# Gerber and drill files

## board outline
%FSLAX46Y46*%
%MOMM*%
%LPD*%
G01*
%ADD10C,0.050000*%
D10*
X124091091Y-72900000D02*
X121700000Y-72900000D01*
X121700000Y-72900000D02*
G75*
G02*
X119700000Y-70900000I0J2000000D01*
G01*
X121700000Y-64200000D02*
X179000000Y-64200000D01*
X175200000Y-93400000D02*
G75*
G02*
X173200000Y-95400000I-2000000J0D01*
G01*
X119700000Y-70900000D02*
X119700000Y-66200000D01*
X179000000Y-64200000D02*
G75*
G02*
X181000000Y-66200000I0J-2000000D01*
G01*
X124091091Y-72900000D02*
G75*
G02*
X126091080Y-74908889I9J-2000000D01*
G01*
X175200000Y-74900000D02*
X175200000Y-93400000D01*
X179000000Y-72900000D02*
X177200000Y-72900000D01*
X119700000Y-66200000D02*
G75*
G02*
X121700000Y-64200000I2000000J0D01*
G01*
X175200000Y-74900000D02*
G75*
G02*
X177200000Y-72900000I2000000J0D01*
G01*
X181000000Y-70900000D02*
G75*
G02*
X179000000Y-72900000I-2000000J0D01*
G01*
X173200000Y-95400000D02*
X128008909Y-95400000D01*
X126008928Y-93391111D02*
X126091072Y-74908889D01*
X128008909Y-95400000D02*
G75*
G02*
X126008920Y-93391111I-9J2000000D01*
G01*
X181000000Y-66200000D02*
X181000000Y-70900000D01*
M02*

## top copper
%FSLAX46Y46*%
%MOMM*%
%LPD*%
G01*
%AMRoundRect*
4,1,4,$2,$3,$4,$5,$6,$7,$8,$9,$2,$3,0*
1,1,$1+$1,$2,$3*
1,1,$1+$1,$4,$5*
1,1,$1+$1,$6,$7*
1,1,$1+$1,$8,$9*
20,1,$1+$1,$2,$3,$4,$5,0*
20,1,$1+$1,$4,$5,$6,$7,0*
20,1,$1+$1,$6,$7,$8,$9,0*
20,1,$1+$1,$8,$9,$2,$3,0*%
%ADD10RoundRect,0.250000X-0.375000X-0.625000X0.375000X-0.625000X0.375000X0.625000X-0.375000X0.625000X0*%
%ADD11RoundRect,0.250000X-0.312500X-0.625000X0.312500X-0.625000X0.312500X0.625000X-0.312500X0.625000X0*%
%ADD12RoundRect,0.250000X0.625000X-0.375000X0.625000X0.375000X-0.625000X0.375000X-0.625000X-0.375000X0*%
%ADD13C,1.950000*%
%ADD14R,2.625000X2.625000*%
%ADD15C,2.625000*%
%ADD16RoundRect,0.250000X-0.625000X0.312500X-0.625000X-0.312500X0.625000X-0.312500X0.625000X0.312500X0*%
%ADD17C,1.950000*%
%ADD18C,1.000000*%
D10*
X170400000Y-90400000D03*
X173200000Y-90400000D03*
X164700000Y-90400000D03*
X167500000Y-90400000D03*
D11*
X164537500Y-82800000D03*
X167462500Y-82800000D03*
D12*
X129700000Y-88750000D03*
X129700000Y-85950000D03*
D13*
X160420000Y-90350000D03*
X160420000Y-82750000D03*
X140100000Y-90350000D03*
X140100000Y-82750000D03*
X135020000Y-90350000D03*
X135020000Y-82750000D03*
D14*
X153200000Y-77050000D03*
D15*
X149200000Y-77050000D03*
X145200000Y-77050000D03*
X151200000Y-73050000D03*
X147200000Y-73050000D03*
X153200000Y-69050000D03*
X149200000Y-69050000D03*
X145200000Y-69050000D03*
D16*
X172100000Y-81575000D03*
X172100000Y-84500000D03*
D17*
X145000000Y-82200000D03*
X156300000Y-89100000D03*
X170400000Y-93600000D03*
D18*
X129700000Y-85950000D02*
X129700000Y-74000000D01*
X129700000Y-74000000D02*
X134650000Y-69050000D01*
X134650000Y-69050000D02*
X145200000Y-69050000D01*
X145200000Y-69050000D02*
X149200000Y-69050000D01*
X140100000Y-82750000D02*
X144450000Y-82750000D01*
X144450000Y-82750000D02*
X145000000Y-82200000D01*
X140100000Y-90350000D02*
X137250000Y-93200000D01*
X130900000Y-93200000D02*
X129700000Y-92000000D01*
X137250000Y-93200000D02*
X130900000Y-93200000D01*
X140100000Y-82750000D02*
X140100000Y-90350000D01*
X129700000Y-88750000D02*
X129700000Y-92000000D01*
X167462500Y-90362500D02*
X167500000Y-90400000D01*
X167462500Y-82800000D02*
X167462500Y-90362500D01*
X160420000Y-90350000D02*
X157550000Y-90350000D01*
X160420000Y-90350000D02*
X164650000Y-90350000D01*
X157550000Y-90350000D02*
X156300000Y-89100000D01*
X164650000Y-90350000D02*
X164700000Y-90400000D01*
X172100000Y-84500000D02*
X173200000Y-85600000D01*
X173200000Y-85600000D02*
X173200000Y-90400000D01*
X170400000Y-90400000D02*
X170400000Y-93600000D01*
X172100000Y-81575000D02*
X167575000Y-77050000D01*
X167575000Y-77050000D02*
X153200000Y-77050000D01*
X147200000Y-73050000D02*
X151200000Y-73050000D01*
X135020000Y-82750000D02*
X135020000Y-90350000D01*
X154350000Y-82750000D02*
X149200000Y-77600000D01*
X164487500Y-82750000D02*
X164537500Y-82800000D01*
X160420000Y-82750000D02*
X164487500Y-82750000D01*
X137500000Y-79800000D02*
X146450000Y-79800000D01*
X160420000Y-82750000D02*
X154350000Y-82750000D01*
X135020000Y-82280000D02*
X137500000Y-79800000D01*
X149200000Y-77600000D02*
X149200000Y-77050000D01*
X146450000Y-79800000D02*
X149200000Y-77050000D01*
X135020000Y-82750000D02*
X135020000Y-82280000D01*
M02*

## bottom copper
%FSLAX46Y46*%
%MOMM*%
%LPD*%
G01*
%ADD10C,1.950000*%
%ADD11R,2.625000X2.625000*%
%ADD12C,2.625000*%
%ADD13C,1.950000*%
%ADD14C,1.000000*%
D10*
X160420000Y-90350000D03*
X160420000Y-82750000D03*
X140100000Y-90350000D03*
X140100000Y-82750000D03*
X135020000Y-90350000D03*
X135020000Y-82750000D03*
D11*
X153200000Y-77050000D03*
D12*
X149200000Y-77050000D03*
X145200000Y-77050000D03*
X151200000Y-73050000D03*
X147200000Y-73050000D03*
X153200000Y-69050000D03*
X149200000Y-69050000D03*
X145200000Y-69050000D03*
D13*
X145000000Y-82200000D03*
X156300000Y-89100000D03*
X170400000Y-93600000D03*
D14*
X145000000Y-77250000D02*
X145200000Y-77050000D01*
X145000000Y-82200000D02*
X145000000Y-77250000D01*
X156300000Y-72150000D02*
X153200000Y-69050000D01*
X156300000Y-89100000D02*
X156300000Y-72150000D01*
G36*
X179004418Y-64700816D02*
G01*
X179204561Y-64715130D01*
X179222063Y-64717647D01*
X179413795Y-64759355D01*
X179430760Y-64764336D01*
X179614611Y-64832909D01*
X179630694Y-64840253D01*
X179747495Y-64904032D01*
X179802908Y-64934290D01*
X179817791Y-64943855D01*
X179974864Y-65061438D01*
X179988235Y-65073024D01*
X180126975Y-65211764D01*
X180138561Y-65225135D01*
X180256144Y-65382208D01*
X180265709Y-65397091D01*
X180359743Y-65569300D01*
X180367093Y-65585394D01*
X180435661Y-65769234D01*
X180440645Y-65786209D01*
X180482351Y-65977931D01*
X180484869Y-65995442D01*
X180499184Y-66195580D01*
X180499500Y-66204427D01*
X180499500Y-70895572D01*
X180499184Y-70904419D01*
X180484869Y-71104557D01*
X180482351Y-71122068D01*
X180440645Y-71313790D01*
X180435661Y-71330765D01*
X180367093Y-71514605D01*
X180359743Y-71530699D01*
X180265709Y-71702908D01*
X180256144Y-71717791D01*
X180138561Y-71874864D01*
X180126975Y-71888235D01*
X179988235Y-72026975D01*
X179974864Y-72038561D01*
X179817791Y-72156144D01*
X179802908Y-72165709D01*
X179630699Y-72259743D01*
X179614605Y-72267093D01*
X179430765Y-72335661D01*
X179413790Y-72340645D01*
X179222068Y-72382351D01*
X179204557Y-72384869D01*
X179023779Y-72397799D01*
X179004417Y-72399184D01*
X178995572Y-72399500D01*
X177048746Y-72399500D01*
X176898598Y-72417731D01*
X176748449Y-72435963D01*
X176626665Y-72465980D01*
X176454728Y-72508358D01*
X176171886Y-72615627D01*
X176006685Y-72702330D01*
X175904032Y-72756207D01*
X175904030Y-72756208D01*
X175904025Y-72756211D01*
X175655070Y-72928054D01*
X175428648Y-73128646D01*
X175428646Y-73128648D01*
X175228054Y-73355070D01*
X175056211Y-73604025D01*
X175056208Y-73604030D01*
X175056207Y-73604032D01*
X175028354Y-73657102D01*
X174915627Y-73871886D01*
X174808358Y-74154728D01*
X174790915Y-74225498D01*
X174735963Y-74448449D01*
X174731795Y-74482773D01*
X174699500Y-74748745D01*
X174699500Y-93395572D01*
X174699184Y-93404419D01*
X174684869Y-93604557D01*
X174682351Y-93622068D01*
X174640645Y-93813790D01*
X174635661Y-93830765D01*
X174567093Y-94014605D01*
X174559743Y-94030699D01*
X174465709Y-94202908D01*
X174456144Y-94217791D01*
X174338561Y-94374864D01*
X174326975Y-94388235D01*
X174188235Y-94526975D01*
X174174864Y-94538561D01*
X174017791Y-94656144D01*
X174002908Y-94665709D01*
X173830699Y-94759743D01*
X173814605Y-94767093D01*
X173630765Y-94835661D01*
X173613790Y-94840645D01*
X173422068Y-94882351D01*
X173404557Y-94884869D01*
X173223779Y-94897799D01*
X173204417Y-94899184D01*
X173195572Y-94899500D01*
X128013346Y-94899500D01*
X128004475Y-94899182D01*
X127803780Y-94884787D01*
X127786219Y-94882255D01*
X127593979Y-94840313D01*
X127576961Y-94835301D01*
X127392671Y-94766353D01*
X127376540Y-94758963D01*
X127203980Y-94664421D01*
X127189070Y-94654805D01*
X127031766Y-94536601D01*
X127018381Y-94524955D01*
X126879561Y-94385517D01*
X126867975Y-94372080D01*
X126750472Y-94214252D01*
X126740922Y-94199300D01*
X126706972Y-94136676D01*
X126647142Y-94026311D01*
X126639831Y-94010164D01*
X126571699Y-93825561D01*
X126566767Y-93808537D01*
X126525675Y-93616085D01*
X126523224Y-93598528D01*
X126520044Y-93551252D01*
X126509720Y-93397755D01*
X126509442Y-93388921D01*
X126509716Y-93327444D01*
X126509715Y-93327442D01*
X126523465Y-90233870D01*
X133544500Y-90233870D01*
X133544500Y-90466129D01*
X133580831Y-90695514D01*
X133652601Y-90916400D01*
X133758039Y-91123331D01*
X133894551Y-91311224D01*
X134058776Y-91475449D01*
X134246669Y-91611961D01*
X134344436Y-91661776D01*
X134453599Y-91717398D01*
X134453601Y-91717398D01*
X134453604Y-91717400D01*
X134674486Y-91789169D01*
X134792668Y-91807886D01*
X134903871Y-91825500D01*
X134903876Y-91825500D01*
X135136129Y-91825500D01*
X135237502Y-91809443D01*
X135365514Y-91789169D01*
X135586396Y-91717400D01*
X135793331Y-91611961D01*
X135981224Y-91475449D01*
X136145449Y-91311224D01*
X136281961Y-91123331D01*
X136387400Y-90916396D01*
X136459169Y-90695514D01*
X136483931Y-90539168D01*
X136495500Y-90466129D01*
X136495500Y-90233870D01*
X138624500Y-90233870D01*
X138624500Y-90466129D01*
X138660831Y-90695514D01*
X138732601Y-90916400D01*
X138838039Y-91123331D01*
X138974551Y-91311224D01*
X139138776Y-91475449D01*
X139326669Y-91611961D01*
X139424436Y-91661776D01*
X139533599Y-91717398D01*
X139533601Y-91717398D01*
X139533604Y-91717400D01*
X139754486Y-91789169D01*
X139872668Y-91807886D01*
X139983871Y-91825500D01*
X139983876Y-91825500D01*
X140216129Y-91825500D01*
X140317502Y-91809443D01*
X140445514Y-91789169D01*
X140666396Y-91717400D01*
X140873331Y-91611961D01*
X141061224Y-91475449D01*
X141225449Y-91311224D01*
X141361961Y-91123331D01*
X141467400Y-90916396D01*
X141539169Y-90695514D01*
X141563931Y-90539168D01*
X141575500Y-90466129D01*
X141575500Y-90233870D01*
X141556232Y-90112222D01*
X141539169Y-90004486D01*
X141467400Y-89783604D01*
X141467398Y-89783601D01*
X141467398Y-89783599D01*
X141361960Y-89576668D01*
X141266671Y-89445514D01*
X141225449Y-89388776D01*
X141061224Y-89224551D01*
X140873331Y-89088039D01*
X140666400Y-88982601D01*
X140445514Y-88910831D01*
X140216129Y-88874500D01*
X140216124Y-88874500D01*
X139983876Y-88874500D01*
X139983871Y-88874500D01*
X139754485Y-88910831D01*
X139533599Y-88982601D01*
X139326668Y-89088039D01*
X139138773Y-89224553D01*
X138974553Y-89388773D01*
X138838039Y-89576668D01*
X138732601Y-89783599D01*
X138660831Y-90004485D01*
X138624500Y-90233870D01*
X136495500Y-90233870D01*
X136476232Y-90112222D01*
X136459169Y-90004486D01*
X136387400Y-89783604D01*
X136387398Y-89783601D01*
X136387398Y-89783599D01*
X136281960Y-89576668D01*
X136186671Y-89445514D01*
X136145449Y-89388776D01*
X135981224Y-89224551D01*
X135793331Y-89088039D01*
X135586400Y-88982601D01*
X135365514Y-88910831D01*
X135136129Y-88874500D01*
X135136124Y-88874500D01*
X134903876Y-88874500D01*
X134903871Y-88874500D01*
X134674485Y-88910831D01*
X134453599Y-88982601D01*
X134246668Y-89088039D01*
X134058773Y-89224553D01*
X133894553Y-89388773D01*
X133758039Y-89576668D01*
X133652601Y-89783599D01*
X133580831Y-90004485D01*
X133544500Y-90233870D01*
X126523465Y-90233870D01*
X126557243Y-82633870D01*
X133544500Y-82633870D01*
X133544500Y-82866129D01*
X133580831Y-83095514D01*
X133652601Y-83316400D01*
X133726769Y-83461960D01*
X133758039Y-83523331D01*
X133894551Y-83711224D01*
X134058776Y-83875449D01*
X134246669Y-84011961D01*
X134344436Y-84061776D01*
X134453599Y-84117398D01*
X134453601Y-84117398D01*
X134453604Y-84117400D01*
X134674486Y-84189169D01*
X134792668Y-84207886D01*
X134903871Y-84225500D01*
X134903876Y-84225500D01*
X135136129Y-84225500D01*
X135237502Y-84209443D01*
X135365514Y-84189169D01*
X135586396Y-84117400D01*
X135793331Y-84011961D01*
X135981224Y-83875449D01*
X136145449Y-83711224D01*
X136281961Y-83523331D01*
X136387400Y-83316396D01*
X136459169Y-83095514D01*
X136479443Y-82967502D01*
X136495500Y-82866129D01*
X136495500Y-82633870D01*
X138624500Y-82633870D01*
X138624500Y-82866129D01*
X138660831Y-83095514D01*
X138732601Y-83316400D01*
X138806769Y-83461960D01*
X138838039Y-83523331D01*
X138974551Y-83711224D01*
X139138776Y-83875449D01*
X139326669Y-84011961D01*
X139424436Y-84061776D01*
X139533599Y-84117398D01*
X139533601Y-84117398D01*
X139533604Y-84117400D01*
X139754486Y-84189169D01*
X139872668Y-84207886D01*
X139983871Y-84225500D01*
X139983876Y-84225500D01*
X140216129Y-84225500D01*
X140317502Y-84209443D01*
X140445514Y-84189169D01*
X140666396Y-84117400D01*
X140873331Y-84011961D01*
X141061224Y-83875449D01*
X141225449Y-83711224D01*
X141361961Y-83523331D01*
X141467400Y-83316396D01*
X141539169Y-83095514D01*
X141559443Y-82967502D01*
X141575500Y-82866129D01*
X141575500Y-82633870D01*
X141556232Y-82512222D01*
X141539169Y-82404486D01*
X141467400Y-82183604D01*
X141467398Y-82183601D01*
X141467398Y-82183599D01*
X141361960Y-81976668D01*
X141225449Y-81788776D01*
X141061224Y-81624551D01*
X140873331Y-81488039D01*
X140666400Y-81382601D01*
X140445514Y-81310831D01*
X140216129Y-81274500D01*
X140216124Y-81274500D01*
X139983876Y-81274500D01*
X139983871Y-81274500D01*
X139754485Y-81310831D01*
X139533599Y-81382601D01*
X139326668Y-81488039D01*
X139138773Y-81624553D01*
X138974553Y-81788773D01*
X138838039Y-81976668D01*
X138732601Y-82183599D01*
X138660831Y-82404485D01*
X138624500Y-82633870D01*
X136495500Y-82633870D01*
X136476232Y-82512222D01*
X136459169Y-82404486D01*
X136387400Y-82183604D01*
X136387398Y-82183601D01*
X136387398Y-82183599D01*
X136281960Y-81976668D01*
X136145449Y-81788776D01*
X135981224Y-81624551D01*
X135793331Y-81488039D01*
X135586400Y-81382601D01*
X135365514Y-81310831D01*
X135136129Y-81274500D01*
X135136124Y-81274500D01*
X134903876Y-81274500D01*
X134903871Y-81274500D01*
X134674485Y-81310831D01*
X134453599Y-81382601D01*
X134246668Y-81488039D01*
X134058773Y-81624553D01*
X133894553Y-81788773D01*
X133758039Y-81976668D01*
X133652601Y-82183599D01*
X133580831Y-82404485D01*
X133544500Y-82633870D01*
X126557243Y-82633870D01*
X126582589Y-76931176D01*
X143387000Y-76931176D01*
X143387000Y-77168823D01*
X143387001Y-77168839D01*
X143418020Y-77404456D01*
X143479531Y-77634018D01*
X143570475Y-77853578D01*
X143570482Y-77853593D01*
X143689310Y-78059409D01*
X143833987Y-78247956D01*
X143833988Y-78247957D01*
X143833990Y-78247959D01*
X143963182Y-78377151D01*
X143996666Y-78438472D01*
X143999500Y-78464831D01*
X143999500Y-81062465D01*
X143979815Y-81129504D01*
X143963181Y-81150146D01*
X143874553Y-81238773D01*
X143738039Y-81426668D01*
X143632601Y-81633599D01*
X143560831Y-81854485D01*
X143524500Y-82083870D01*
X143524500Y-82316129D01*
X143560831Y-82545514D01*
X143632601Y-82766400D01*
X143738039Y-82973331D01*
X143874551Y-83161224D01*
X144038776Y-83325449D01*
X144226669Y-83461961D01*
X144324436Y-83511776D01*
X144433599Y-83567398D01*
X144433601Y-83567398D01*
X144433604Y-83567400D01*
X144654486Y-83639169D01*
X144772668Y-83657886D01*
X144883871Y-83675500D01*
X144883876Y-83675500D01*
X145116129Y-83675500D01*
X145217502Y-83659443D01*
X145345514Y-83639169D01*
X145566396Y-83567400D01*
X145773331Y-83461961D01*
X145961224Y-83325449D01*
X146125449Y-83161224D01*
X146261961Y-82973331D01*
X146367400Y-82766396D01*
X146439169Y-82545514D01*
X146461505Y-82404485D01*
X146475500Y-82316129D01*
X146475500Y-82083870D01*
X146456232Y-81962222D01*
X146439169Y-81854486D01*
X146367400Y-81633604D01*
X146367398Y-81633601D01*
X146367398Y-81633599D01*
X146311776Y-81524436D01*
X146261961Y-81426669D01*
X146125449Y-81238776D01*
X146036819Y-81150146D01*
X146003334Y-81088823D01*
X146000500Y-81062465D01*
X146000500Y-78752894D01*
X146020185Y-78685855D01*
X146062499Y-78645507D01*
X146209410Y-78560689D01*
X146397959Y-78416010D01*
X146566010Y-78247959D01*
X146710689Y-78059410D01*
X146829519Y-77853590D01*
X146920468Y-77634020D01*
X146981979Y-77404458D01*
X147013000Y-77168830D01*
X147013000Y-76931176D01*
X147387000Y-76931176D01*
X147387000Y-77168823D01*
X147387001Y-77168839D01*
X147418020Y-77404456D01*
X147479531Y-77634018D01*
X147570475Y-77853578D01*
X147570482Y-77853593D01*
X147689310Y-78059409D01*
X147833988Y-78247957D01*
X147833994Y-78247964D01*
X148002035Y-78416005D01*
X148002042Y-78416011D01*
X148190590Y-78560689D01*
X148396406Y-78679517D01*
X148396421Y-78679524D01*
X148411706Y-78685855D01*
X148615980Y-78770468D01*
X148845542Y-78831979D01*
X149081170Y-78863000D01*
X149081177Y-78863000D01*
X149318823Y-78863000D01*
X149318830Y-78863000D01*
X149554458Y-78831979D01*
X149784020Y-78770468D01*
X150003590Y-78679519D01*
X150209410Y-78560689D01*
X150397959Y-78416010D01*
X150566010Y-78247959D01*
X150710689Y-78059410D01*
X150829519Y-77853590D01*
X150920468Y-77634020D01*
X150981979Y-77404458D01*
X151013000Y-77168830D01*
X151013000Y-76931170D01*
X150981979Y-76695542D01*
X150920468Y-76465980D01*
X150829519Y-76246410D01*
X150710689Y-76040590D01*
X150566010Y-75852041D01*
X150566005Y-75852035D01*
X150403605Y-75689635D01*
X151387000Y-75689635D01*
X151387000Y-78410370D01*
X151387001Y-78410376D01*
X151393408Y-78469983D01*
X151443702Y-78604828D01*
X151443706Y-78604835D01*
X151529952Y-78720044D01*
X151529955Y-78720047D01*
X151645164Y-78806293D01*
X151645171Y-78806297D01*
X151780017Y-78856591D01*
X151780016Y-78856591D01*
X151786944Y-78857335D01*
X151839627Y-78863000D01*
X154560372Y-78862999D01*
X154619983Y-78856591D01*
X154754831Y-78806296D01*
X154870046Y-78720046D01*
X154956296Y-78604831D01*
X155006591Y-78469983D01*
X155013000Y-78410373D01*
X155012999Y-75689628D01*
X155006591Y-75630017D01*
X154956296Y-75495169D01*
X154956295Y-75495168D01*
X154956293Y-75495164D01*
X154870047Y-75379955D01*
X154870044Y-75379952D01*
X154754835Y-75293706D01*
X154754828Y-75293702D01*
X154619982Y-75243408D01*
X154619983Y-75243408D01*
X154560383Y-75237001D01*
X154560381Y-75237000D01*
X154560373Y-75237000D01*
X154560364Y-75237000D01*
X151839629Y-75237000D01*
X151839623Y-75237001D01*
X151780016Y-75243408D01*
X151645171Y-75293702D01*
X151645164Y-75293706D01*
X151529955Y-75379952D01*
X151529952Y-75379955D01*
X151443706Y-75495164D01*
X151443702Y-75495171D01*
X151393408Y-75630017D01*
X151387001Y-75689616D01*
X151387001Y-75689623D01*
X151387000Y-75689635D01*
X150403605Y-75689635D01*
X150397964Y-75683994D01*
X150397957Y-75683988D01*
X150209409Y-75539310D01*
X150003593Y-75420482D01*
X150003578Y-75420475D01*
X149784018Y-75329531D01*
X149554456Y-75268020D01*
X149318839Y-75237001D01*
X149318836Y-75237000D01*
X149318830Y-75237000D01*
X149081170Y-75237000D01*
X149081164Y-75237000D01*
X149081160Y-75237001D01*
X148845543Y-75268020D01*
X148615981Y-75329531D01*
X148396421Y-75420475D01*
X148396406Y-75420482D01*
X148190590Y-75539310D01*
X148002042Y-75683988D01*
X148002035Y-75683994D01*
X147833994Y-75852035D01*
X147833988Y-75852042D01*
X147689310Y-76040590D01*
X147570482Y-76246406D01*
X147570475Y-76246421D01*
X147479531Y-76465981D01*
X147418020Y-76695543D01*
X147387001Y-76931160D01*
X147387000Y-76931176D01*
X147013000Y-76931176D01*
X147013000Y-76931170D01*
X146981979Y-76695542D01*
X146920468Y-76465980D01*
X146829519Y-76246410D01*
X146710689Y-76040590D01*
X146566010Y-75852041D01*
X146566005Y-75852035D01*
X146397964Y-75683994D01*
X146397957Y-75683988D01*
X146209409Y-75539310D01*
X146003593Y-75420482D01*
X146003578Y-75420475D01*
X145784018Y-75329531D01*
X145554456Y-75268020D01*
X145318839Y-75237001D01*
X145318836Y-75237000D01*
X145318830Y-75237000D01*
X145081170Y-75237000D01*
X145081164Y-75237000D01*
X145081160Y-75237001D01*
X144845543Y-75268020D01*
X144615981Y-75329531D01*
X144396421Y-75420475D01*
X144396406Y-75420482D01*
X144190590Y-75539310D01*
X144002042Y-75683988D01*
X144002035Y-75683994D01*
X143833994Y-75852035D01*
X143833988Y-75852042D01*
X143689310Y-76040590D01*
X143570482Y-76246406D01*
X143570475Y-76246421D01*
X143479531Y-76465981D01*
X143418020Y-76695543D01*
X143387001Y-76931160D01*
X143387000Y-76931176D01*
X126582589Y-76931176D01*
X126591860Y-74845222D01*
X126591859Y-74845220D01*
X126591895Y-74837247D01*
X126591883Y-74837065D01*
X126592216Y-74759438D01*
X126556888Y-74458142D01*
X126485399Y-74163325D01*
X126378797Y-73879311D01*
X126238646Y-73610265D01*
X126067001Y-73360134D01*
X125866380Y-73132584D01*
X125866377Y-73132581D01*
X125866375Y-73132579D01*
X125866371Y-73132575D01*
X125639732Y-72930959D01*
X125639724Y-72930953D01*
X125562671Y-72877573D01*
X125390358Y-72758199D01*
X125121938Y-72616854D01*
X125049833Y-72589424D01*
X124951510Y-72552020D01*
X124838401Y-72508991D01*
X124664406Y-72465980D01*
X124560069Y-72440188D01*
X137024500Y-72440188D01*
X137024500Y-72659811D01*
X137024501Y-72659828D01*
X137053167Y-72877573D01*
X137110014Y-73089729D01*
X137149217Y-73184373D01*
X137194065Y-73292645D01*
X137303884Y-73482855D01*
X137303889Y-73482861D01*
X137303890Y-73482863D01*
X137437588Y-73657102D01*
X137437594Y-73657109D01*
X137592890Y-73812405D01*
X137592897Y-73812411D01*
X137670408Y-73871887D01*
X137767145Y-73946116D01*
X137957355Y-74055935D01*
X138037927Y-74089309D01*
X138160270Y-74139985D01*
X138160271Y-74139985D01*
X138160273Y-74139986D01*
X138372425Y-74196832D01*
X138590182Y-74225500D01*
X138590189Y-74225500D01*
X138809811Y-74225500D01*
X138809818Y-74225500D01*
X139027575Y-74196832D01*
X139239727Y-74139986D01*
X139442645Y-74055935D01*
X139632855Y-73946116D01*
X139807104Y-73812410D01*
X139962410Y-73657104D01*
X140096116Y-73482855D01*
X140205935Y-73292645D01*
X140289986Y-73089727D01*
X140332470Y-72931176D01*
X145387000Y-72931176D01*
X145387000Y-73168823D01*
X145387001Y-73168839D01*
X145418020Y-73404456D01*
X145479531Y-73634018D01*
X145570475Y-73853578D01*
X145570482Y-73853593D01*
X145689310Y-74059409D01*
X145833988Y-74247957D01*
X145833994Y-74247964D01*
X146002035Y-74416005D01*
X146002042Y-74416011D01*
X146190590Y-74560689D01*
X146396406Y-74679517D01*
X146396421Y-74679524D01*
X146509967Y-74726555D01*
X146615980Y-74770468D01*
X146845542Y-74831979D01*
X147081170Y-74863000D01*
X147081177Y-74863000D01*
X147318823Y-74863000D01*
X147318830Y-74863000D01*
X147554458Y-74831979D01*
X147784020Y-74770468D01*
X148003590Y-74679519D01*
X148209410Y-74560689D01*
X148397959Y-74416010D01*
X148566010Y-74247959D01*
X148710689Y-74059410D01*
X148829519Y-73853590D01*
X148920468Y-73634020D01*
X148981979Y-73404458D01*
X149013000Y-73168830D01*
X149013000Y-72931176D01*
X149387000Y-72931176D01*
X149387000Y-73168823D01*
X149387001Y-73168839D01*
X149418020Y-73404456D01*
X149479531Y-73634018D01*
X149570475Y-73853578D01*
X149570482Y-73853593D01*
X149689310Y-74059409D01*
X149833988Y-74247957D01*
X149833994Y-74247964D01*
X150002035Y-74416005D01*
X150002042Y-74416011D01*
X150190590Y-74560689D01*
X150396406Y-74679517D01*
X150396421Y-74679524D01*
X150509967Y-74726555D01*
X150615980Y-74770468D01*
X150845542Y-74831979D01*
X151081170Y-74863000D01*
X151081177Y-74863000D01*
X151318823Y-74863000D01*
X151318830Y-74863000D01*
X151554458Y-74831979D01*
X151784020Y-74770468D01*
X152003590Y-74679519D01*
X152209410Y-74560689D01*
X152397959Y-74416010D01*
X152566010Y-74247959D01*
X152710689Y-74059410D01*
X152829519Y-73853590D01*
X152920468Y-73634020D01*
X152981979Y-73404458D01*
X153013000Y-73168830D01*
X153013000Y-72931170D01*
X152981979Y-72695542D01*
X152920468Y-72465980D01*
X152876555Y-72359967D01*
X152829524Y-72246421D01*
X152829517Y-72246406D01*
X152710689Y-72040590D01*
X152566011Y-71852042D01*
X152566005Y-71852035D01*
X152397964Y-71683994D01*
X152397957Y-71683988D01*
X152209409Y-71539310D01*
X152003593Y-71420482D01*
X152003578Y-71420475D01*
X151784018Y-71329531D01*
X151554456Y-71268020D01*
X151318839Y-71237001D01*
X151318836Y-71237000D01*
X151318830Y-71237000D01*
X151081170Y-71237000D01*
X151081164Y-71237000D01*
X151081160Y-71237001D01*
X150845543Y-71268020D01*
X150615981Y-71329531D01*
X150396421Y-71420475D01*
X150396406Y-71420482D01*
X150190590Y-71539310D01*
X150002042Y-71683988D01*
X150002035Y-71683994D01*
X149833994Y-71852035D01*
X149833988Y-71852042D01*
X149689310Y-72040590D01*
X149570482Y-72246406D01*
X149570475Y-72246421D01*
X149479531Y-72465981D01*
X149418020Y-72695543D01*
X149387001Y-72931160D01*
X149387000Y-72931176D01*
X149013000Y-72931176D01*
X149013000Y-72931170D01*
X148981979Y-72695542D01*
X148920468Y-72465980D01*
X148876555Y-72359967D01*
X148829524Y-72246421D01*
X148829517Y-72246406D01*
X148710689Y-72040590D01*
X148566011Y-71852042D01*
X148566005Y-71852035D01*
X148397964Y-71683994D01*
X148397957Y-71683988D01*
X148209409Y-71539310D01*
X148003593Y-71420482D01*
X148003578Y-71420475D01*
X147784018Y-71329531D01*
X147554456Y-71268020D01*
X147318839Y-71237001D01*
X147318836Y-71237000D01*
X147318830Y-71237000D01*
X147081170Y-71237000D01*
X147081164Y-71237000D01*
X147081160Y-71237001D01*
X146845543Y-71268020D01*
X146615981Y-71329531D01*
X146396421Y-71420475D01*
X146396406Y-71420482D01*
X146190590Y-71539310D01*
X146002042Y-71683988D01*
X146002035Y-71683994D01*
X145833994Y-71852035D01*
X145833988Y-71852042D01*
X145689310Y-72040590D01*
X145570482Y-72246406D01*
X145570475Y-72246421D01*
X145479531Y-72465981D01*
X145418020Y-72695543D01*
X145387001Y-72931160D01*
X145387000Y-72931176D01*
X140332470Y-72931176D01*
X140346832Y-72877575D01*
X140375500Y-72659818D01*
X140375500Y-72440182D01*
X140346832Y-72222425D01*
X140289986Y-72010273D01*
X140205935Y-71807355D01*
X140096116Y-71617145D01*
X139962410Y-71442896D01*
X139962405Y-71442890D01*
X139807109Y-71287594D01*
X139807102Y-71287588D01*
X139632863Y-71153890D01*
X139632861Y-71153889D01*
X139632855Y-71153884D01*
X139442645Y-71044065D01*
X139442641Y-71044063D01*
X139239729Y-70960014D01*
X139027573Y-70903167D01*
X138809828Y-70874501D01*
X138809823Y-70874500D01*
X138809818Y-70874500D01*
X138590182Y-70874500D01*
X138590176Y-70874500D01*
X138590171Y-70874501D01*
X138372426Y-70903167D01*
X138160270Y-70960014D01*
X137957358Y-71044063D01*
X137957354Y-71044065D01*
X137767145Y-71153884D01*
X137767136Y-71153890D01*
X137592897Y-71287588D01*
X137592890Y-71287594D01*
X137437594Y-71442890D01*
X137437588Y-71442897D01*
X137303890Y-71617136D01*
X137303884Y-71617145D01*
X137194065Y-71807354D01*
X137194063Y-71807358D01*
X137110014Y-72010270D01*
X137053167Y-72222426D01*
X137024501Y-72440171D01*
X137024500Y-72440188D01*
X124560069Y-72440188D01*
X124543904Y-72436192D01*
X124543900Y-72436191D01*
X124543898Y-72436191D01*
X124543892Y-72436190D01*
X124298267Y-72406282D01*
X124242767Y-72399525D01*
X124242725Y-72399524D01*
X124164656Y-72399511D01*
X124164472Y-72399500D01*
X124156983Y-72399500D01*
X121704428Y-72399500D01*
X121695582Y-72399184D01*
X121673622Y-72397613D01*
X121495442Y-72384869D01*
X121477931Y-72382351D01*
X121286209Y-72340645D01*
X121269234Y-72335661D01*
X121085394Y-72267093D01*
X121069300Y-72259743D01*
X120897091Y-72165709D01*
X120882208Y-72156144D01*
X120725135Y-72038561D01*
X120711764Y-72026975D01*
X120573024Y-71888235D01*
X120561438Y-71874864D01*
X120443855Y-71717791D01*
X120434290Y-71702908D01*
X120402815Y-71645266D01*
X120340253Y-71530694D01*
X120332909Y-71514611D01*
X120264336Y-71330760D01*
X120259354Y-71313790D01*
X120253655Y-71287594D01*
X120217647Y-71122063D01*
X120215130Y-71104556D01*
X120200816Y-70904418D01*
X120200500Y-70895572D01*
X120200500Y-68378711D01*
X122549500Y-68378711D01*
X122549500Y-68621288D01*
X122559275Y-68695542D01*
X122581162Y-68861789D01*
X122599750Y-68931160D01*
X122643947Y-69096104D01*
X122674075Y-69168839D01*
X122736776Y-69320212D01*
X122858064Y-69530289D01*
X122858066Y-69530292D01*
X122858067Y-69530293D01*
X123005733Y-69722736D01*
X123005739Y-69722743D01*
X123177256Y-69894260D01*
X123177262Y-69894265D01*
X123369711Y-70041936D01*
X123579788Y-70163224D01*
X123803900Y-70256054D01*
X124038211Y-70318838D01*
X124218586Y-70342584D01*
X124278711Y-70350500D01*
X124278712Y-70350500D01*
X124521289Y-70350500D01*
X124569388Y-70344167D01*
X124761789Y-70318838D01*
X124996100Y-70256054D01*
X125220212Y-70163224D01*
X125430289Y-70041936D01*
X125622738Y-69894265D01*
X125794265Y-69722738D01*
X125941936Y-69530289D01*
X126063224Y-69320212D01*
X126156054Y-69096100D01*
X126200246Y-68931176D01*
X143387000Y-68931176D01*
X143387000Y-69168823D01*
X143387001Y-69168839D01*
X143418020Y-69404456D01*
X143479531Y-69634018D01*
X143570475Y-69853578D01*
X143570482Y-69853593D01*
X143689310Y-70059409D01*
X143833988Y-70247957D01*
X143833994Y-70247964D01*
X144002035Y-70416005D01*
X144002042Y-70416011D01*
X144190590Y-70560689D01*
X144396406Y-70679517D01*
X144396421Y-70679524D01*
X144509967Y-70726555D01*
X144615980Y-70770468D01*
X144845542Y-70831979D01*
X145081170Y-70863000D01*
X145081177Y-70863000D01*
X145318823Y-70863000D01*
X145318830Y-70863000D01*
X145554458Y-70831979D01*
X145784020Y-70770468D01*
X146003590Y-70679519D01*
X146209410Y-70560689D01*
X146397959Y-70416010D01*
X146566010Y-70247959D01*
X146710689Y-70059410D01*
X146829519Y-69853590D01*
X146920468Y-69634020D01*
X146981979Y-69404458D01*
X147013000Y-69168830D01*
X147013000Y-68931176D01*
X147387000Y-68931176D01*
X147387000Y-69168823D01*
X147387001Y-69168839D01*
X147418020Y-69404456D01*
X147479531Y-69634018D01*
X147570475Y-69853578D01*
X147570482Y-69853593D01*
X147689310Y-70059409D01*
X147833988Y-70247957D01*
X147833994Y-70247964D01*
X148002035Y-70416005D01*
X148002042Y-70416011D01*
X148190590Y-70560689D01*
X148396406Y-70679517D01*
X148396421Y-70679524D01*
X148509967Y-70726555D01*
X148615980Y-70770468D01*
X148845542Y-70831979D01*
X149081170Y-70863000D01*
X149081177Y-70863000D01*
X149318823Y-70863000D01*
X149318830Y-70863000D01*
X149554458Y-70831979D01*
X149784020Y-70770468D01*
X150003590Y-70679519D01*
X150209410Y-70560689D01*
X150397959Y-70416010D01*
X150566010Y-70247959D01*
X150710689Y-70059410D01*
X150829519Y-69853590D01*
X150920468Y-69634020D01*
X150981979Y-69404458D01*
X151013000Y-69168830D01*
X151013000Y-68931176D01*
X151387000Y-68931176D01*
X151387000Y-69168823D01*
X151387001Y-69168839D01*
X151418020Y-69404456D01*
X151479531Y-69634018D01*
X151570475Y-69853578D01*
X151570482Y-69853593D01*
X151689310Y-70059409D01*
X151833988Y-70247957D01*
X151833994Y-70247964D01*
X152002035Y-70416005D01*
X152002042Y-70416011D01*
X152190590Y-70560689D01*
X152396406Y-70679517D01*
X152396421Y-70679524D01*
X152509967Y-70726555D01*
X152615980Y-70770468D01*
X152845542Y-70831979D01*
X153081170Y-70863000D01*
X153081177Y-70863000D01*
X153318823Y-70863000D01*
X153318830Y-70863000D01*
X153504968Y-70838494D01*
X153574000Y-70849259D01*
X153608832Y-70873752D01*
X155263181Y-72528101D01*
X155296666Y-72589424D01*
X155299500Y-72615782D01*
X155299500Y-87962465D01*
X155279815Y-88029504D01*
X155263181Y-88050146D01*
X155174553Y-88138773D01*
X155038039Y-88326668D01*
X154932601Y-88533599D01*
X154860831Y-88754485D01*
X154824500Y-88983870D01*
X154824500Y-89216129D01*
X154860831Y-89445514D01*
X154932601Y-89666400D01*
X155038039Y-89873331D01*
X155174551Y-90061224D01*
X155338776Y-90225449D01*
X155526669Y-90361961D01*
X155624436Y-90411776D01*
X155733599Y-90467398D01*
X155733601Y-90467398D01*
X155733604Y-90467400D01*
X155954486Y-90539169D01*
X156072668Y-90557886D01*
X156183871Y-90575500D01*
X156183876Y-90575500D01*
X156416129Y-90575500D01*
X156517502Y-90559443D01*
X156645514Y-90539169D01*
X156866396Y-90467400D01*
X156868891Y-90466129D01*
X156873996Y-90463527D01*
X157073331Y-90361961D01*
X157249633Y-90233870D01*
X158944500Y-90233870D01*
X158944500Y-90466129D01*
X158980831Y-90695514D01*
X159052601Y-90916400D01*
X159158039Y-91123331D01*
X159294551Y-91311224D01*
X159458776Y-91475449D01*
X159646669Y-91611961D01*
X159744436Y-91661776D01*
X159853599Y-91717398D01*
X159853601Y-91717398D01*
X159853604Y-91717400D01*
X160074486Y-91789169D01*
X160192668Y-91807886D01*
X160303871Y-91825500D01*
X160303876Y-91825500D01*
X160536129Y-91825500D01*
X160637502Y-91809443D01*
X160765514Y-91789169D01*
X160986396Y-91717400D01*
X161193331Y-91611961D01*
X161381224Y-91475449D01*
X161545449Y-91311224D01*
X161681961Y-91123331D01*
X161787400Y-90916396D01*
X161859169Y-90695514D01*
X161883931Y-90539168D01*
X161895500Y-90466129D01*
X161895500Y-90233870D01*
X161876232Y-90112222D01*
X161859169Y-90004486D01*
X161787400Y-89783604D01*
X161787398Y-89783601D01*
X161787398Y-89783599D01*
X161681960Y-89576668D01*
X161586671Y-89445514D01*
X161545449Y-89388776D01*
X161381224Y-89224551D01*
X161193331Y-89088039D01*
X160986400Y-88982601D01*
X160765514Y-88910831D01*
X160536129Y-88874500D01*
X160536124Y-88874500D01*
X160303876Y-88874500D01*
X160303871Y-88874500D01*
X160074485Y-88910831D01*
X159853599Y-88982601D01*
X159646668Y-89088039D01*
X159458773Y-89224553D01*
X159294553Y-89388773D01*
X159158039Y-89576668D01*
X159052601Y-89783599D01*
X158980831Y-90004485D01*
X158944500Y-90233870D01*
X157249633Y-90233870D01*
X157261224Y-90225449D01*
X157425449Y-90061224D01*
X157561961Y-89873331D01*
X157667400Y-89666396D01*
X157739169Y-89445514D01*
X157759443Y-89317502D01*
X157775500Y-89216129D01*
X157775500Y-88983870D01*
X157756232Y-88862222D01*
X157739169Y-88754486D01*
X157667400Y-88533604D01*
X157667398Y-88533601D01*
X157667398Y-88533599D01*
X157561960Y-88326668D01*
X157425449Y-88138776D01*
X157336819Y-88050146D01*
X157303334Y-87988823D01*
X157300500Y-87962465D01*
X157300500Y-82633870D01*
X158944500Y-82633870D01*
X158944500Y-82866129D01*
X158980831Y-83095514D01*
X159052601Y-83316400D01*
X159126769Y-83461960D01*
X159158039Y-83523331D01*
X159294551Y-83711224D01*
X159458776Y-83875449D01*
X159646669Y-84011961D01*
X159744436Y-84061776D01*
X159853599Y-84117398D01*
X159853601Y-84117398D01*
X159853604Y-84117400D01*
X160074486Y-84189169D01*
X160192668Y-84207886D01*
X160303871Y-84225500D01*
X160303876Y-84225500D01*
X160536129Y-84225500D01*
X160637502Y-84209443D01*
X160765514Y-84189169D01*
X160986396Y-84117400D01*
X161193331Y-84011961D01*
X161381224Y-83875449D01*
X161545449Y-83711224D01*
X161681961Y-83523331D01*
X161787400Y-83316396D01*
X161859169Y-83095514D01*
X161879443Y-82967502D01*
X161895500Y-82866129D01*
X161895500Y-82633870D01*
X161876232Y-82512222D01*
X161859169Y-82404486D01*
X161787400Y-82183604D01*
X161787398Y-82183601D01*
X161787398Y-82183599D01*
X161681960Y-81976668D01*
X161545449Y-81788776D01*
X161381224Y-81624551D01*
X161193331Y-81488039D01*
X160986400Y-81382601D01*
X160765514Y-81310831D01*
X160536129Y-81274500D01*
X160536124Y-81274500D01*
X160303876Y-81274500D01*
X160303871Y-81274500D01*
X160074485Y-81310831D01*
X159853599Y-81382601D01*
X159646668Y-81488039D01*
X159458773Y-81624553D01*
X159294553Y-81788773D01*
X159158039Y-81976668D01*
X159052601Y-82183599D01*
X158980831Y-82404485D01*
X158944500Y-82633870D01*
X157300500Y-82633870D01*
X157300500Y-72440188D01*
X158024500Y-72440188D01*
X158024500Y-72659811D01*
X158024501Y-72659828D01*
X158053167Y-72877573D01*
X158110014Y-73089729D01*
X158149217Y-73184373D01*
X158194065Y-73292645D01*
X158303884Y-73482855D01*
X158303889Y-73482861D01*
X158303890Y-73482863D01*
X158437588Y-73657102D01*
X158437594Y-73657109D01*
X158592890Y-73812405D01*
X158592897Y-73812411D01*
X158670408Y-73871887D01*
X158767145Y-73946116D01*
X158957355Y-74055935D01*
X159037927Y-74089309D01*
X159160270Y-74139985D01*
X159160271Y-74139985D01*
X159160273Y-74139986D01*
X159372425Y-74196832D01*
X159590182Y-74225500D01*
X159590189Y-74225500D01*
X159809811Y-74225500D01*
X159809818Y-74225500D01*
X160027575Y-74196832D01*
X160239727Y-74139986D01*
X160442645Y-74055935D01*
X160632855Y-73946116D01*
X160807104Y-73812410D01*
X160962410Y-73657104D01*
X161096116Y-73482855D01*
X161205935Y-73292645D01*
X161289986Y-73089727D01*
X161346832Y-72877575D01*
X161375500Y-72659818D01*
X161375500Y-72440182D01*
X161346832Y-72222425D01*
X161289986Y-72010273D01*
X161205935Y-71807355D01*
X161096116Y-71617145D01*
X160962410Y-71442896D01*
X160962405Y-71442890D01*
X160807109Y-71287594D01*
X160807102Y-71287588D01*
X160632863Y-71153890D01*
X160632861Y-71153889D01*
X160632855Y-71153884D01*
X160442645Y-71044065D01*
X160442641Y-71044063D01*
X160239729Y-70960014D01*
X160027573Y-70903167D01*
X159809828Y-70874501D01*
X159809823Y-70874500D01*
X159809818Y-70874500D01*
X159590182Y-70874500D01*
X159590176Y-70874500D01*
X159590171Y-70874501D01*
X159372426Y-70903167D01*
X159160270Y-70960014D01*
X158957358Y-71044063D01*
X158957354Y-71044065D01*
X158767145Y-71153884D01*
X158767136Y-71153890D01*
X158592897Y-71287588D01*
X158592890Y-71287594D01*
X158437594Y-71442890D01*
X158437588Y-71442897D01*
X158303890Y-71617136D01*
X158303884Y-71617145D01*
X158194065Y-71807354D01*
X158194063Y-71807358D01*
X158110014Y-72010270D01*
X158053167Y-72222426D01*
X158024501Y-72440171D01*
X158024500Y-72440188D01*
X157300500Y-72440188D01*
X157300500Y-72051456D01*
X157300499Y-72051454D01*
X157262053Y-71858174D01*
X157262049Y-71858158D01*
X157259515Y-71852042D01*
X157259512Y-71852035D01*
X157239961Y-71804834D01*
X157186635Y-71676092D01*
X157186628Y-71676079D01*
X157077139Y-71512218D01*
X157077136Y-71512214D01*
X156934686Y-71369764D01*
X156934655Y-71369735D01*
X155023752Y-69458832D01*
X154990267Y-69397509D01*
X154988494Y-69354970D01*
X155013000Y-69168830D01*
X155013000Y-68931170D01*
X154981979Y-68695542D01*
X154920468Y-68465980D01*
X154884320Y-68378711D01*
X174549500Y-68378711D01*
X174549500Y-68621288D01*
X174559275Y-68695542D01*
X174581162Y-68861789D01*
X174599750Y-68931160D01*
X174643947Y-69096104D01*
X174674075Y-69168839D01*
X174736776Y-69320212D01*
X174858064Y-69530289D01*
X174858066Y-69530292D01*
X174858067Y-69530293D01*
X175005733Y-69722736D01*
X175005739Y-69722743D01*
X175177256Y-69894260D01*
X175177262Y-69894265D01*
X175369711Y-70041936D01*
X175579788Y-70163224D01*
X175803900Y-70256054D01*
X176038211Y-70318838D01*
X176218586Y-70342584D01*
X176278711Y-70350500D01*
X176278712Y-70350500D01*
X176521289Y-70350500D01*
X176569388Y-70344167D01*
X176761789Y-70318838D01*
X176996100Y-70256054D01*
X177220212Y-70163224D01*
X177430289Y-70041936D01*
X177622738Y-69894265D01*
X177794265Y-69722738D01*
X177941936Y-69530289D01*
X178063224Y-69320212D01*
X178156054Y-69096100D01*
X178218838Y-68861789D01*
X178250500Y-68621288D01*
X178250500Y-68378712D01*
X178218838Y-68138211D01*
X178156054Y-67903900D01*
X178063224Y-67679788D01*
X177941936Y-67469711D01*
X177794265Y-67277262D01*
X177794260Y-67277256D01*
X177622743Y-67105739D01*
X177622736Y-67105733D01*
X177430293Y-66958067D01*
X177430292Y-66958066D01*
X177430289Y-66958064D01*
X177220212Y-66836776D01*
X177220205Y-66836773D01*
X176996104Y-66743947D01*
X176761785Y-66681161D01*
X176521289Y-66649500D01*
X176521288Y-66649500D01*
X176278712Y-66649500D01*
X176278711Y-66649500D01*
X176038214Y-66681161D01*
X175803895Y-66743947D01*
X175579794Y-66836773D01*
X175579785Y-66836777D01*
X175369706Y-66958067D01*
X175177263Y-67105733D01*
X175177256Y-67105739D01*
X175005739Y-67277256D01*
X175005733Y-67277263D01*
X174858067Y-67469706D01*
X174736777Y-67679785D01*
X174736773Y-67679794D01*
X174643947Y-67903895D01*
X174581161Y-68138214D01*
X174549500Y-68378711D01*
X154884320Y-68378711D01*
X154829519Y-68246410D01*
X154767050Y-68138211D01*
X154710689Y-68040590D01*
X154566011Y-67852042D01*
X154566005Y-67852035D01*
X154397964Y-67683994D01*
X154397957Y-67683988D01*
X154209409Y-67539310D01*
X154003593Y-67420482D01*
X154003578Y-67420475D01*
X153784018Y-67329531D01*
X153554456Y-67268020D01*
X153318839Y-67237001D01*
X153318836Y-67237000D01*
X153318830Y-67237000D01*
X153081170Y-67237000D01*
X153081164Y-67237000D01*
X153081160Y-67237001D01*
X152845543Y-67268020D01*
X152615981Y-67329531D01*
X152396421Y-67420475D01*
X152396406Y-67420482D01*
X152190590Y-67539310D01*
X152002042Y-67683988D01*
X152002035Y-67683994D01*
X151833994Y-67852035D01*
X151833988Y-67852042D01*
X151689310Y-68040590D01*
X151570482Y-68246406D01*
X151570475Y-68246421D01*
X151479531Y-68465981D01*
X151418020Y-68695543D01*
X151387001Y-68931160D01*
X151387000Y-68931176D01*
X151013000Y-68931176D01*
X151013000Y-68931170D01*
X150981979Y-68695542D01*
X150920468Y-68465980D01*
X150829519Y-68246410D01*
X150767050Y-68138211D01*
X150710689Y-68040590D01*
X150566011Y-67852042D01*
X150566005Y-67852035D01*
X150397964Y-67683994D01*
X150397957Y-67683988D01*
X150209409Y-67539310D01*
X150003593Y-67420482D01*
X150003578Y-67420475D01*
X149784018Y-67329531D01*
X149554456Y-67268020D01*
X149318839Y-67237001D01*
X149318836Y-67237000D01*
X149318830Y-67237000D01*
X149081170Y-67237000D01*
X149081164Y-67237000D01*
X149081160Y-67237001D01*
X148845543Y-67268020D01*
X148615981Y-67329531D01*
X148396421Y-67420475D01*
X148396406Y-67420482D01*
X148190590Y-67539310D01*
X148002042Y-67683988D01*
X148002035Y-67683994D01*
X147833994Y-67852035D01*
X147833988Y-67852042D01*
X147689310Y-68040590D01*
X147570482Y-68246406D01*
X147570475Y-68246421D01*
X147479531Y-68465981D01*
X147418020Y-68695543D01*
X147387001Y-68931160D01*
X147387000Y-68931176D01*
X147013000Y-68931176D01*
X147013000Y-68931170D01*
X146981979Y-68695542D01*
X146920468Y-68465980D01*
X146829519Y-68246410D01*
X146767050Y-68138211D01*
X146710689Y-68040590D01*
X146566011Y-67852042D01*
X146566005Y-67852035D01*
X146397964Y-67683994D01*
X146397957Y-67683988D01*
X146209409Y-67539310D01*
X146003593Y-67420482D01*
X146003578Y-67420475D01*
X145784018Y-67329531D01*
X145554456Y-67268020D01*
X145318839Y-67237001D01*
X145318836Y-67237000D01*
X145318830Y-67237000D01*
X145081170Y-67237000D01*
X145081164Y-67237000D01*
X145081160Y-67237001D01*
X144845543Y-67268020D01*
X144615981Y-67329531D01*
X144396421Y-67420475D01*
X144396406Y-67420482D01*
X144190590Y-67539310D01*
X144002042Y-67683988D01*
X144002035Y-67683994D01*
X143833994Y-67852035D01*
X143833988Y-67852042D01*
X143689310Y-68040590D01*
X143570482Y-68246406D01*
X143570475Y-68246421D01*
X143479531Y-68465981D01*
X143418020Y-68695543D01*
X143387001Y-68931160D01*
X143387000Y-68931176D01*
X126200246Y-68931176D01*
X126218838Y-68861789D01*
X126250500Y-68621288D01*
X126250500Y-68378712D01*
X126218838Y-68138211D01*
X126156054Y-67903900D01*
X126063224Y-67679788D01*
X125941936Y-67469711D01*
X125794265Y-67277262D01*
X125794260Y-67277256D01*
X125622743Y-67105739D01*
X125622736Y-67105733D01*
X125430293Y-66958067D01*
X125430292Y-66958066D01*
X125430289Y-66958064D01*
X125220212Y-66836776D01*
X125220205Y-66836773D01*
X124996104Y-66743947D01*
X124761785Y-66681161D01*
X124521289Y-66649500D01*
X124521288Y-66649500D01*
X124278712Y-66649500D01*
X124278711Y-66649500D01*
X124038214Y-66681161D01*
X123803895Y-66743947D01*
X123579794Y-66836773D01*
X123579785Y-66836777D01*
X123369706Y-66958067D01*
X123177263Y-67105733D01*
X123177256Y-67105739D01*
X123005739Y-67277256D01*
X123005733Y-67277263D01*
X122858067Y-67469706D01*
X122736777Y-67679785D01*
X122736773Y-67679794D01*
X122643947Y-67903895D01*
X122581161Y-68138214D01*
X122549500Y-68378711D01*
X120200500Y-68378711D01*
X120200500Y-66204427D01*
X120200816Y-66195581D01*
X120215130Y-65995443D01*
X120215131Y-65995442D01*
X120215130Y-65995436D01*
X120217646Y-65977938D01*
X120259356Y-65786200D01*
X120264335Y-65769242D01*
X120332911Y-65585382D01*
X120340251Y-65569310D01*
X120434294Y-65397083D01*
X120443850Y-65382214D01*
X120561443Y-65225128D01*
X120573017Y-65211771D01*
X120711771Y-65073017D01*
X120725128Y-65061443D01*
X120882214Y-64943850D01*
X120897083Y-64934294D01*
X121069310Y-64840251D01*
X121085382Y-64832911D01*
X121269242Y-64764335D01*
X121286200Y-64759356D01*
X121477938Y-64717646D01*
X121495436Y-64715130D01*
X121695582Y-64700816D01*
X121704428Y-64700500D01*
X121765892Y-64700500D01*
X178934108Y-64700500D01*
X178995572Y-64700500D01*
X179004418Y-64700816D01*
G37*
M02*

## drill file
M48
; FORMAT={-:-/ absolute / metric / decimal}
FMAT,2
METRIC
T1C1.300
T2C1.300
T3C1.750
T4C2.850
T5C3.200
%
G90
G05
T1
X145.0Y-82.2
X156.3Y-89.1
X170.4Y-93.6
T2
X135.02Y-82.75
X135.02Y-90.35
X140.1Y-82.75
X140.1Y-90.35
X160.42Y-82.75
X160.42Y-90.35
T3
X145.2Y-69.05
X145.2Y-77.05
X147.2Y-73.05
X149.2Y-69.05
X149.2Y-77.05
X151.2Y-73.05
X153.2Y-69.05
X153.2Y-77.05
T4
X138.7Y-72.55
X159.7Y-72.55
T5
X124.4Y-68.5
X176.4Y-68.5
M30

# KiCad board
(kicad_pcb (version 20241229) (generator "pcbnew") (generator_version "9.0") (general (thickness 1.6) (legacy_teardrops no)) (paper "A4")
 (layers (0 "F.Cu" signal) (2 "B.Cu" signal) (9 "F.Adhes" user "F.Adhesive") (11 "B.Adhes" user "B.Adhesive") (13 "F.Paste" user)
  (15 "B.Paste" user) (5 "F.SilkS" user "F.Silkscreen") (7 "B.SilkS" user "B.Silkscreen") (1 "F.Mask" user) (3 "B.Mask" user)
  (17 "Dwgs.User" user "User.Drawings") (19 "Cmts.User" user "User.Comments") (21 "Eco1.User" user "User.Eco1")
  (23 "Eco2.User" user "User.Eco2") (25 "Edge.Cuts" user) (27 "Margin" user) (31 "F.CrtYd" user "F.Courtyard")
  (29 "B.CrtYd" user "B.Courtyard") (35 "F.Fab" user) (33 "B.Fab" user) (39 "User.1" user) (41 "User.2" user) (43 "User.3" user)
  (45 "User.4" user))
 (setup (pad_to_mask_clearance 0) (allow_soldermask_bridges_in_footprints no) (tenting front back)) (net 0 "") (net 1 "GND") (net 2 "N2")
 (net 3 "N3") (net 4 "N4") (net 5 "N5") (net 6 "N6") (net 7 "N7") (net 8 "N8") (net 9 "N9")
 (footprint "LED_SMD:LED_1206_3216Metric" (layer "F.Cu") (at 171.8 90.4)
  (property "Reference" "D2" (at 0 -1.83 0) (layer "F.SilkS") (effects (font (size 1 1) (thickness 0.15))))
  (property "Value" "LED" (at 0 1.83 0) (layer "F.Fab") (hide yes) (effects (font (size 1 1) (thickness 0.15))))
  (pad "1" smd roundrect (at -1.4 0) (size 1.25 1.75) (layers "F.Cu" "F.Mask" "F.Paste") (roundrect_rratio 0.2) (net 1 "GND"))
  (pad "2" smd roundrect (at 1.4 0) (size 1.25 1.75) (layers "F.Cu" "F.Mask" "F.Paste") (roundrect_rratio 0.2) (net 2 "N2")))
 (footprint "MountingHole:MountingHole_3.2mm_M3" (layer "F.Cu") (at 176.4 68.5)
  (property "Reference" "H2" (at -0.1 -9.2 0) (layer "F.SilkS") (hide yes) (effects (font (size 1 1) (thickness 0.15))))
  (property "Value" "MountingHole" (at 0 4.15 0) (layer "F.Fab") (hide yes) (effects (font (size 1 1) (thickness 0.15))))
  (pad "" np_thru_hole circle (at 0 0) (size 3.2 3.2) (drill 3.2) (layers "*.Cu" "*.Mask")))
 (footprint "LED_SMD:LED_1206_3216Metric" (layer "F.Cu") (at 166.1 90.4)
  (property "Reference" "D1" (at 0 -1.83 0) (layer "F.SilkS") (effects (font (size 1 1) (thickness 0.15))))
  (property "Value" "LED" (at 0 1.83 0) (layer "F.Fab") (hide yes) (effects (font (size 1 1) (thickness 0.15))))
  (pad "1" smd roundrect (at -1.4 0) (size 1.25 1.75) (layers "F.Cu" "F.Mask" "F.Paste") (roundrect_rratio 0.2) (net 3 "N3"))
  (pad "2" smd roundrect (at 1.4 0) (size 1.25 1.75) (layers "F.Cu" "F.Mask" "F.Paste") (roundrect_rratio 0.2) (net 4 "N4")))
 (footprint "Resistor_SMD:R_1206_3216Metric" (layer "F.Cu") (at 166 82.8)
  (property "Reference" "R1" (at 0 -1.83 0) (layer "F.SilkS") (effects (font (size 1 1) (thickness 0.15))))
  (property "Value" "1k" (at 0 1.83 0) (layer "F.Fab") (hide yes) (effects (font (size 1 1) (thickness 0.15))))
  (pad "1" smd roundrect (at -1.4625 0) (size 1.125 1.75) (layers "F.Cu" "F.Mask" "F.Paste") (roundrect_rratio 0.222222) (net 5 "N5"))
  (pad "2" smd roundrect (at 1.4625 0) (size 1.125 1.75) (layers "F.Cu" "F.Mask" "F.Paste") (roundrect_rratio 0.222222) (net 4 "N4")))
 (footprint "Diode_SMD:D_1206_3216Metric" (layer "F.Cu") (at 129.7 87.35 90)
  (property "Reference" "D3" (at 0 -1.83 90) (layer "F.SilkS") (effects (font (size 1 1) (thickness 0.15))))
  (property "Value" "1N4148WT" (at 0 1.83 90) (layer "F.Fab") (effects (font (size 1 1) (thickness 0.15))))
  (pad "1" smd roundrect (at -1.4 0 90) (size 1.25 1.75) (layers "F.Cu" "F.Mask" "F.Paste") (roundrect_rratio 0.2) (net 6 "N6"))
  (pad "2" smd roundrect (at 1.4 0 90) (size 1.25 1.75) (layers "F.Cu" "F.Mask" "F.Paste") (roundrect_rratio 0.2) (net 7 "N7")))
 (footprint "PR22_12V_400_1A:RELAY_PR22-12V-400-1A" (layer "F.Cu") (at 148.42 86.55 180)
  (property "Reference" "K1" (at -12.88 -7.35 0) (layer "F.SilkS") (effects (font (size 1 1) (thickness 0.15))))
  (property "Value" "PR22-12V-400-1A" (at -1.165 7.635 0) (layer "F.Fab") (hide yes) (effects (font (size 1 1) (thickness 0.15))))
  (pad "A1" thru_hole circle (at -12 -3.8 180) (size 1.95 1.95) (drill 1.3) (layers "*.Cu" "*.Mask") (remove_unused_layers no) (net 3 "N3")
   (solder_mask_margin 0.102))
  (pad "A2" thru_hole circle (at -12 3.8 180) (size 1.95 1.95) (drill 1.3) (layers "*.Cu" "*.Mask") (remove_unused_layers no) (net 5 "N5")
   (solder_mask_margin 0.102))
  (pad "COM_1" thru_hole circle (at 8.32 -3.8 180) (size 1.95 1.95) (drill 1.3) (layers "*.Cu" "*.Mask") (remove_unused_layers no)
   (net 6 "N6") (solder_mask_margin 0.102))
  (pad "COM_2" thru_hole circle (at 8.32 3.8 180) (size 1.95 1.95) (drill 1.3) (layers "*.Cu" "*.Mask") (remove_unused_layers no)
   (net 6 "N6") (solder_mask_margin 0.102))
  (pad "NO_1" thru_hole circle (at 13.4 -3.8 180) (size 1.95 1.95) (drill 1.3) (layers "*.Cu" "*.Mask") (remove_unused_layers no)
   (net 5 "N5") (solder_mask_margin 0.102))
  (pad "NO_2" thru_hole circle (at 13.4 3.8 180) (size 1.95 1.95) (drill 1.3) (layers "*.Cu" "*.Mask") (remove_unused_layers no)
   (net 5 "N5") (solder_mask_margin 0.102)))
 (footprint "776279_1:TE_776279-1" (layer "F.Cu") (at 149.2 73.05 180)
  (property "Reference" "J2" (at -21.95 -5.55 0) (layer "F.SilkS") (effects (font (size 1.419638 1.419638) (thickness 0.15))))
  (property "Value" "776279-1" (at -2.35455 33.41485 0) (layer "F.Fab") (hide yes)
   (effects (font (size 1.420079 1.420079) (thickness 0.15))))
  (pad "" np_thru_hole circle (at -10.5 0.5 180) (size 2.85 2.85) (drill 2.85) (layers "*.Cu" "*.Mask"))
  (pad "" np_thru_hole circle (at 10.5 0.5 180) (size 2.85 2.85) (drill 2.85) (layers "*.Cu" "*.Mask"))
  (pad "1" thru_hole rect (at -4 -4 180) (size 2.625 2.625) (drill 1.75) (layers "*.Cu" "*.Mask") (remove_unused_layers no) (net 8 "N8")
   (solder_mask_margin 0.102))
  (pad "2" thru_hole circle (at 0 -4 180) (size 2.625 2.625) (drill 1.75) (layers "*.Cu" "*.Mask") (remove_unused_layers no) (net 5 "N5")
   (solder_mask_margin 0.102))
  (pad "3" thru_hole circle (at 4 -4 180) (size 2.625 2.625) (drill 1.75) (layers "*.Cu" "*.Mask") (remove_unused_layers no) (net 6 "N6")
   (solder_mask_margin 0.102))
  (pad "4" thru_hole circle (at -2 0 180) (size 2.625 2.625) (drill 1.75) (layers "*.Cu" "*.Mask") (remove_unused_layers no) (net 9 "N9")
   (solder_mask_margin 0.102))
  (pad "5" thru_hole circle (at 2 0 180) (size 2.625 2.625) (drill 1.75) (layers "*.Cu" "*.Mask") (remove_unused_layers no) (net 9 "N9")
   (solder_mask_margin 0.102))
  (pad "6" thru_hole circle (at -4 4 180) (size 2.625 2.625) (drill 1.75) (layers "*.Cu" "*.Mask") (remove_unused_layers no) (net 3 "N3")
   (solder_mask_margin 0.102))
  (pad "7" thru_hole circle (at 0 4 180) (size 2.625 2.625) (drill 1.75) (layers "*.Cu" "*.Mask") (remove_unused_layers no) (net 7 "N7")
   (solder_mask_margin 0.102))
  (pad "8" thru_hole circle (at 4 4 180) (size 2.625 2.625) (drill 1.75) (layers "*.Cu" "*.Mask") (remove_unused_layers no) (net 7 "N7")
   (solder_mask_margin 0.102)))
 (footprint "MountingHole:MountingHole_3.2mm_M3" (layer "F.Cu") (at 124.4 68.5)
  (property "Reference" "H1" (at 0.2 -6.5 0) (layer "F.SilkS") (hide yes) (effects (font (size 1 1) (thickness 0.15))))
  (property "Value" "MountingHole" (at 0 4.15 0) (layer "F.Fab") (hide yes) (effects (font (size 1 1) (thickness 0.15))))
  (pad "" np_thru_hole circle (at 0 0) (size 3.2 3.2) (drill 3.2) (layers "*.Cu" "*.Mask")))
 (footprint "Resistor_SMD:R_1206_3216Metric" (layer "F.Cu") (at 172.1 83.0375 -90)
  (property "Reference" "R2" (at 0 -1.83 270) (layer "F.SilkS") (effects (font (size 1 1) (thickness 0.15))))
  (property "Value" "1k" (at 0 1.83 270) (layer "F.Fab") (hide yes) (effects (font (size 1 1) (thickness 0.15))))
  (pad "1" smd roundrect (at -1.4625 0 270) (size 1.125 1.75) (layers "F.Cu" "F.Mask" "F.Paste") (roundrect_rratio 0.222222) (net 8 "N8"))
  (pad "2" smd roundrect (at 1.4625 0 270) (size 1.125 1.75) (layers "F.Cu" "F.Mask" "F.Paste") (roundrect_rratio 0.222222) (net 2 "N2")))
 (gr_line (start 124.091091 72.9) (end 121.7 72.9) (stroke (width 0.05) (type default)) (layer "Edge.Cuts"))
 (gr_arc (start 121.7 72.9) (mid 120.285786 72.314214) (end 119.7 70.9) (stroke (width 0.05) (type default)) (layer "Edge.Cuts"))
 (gr_line (start 121.7 64.2) (end 179 64.2) (stroke (width 0.05) (type default)) (layer "Edge.Cuts"))
 (gr_arc (start 175.2 93.4) (mid 174.614214 94.814214) (end 173.2 95.4) (stroke (width 0.05) (type default)) (layer "Edge.Cuts"))
 (gr_line (start 119.7 70.9) (end 119.7 66.2) (stroke (width 0.05) (type default)) (layer "Edge.Cuts"))
 (gr_arc (start 179 64.2) (mid 180.414214 64.785786) (end 181 66.2) (stroke (width 0.05) (type default)) (layer "Edge.Cuts"))
 (gr_arc (start 124.091091 72.9) (mid 125.50845 73.488929) (end 126.091072 74.908889) (stroke (width 0.05) (type default))
  (layer "Edge.Cuts"))
 (gr_line (start 175.2 74.9) (end 175.2 93.4) (stroke (width 0.05) (type default)) (layer "Edge.Cuts"))
 (gr_line (start 179 72.9) (end 177.2 72.9) (stroke (width 0.05) (type default)) (layer "Edge.Cuts"))
 (gr_arc (start 119.7 66.2) (mid 120.285786 64.785786) (end 121.7 64.2) (stroke (width 0.05) (type default)) (layer "Edge.Cuts"))
 (gr_arc (start 175.2 74.9) (mid 175.785786 73.485786) (end 177.2 72.9) (stroke (width 0.05) (type default)) (layer "Edge.Cuts"))
 (gr_arc (start 181 70.9) (mid 180.414214 72.314214) (end 179 72.9) (stroke (width 0.05) (type default)) (layer "Edge.Cuts"))
 (gr_line (start 173.2 95.4) (end 128.008909 95.4) (stroke (width 0.05) (type default)) (layer "Edge.Cuts"))
 (gr_line (start 126.008928 93.391111) (end 126.091072 74.908889) (stroke (width 0.05) (type default)) (layer "Edge.Cuts"))
 (gr_arc (start 128.008909 95.4) (mid 126.591556 94.811067) (end 126.008928 93.391111) (stroke (width 0.05) (type default))
  (layer "Edge.Cuts"))
 (gr_line (start 181 66.2) (end 181 70.9) (stroke (width 0.05) (type default)) (layer "Edge.Cuts"))
 (segment (start 129.7 85.95) (end 129.7 74) (width 1) (layer "F.Cu") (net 7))
 (segment (start 129.7 74) (end 134.65 69.05) (width 1) (layer "F.Cu") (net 7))
 (segment (start 134.65 69.05) (end 145.2 69.05) (width 1) (layer "F.Cu") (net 7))
 (segment (start 145.2 69.05) (end 149.2 69.05) (width 1) (layer "F.Cu") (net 7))
 (segment (start 140.1 82.75) (end 144.45 82.75) (width 1) (layer "F.Cu") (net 6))
 (segment (start 144.45 82.75) (end 145 82.2) (width 1) (layer "F.Cu") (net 6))
 (segment (start 140.1 90.35) (end 137.25 93.2) (width 1) (layer "F.Cu") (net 6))
 (segment (start 130.9 93.2) (end 129.7 92) (width 1) (layer "F.Cu") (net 6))
 (segment (start 137.25 93.2) (end 130.9 93.2) (width 1) (layer "F.Cu") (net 6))
 (segment (start 140.1 82.75) (end 140.1 90.35) (width 1) (layer "F.Cu") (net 6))
 (segment (start 129.7 88.75) (end 129.7 92) (width 1) (layer "F.Cu") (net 6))
 (via (at 145 82.2) (size 1.95) (drill 1.3) (layers "F.Cu" "B.Cu") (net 6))
 (segment (start 145 77.25) (end 145.2 77.05) (width 1) (layer "B.Cu") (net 6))
 (segment (start 145 82.2) (end 145 77.25) (width 1) (layer "B.Cu") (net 6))
 (segment (start 167.4625 90.3625) (end 167.5 90.4) (width 1) (layer "F.Cu") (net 4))
 (segment (start 167.4625 82.8) (end 167.4625 90.3625) (width 1) (layer "F.Cu") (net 4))
 (segment (start 160.42 90.35) (end 157.55 90.35) (width 1) (layer "F.Cu") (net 3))
 (segment (start 160.42 90.35) (end 164.65 90.35) (width 1) (layer "F.Cu") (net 3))
 (segment (start 157.55 90.35) (end 156.3 89.1) (width 1) (layer "F.Cu") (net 3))
 (segment (start 164.65 90.35) (end 164.7 90.4) (width 1) (layer "F.Cu") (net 3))
 (via (at 156.3 89.1) (size 1.95) (drill 1.3) (layers "F.Cu" "B.Cu") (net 3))
 (segment (start 156.3 72.15) (end 153.2 69.05) (width 1) (layer "B.Cu") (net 3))
 (segment (start 156.3 89.1) (end 156.3 72.15) (width 1) (layer "B.Cu") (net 3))
 (segment (start 172.1 84.5) (end 173.2 85.6) (width 1) (layer "F.Cu") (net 2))
 (segment (start 173.2 85.6) (end 173.2 90.4) (width 1) (layer "F.Cu") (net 2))
 (segment (start 170.4 90.4) (end 170.4 93.6) (width 1) (layer "F.Cu") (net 1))
 (via (at 170.4 93.6) (size 1.95) (drill 1.3) (layers "F.Cu" "B.Cu") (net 1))
 (segment (start 172.1 81.575) (end 167.575 77.05) (width 1) (layer "F.Cu") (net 8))
 (segment (start 167.575 77.05) (end 153.2 77.05) (width 1) (layer "F.Cu") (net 8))
 (segment (start 147.2 73.05) (end 151.2 73.05) (width 1) (layer "F.Cu") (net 9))
 (segment (start 135.02 82.75) (end 135.02 90.35) (width 1) (layer "F.Cu") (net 5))
 (segment (start 154.35 82.75) (end 149.2 77.6) (width 1) (layer "F.Cu") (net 5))
 (segment (start 164.4875 82.75) (end 164.5375 82.8) (width 1) (layer "F.Cu") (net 5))
 (segment (start 160.42 82.75) (end 164.4875 82.75) (width 1) (layer "F.Cu") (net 5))
 (segment (start 137.5 79.8) (end 146.45 79.8) (width 1) (layer "F.Cu") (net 5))
 (segment (start 160.42 82.75) (end 154.35 82.75) (width 1) (layer "F.Cu") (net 5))
 (segment (start 135.02 82.28) (end 137.5 79.8) (width 1) (layer "F.Cu") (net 5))
 (segment (start 149.2 77.6) (end 149.2 77.05) (width 1) (layer "F.Cu") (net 5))
 (segment (start 146.45 79.8) (end 149.2 77.05) (width 1) (layer "F.Cu") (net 5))
 (segment (start 135.02 82.75) (end 135.02 82.28) (width 1) (layer "F.Cu") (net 5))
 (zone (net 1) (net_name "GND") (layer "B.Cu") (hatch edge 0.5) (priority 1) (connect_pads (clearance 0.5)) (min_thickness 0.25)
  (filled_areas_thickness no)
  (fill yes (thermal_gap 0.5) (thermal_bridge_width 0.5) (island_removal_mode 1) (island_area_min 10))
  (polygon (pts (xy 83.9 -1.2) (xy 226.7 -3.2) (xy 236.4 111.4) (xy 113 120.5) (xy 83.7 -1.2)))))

